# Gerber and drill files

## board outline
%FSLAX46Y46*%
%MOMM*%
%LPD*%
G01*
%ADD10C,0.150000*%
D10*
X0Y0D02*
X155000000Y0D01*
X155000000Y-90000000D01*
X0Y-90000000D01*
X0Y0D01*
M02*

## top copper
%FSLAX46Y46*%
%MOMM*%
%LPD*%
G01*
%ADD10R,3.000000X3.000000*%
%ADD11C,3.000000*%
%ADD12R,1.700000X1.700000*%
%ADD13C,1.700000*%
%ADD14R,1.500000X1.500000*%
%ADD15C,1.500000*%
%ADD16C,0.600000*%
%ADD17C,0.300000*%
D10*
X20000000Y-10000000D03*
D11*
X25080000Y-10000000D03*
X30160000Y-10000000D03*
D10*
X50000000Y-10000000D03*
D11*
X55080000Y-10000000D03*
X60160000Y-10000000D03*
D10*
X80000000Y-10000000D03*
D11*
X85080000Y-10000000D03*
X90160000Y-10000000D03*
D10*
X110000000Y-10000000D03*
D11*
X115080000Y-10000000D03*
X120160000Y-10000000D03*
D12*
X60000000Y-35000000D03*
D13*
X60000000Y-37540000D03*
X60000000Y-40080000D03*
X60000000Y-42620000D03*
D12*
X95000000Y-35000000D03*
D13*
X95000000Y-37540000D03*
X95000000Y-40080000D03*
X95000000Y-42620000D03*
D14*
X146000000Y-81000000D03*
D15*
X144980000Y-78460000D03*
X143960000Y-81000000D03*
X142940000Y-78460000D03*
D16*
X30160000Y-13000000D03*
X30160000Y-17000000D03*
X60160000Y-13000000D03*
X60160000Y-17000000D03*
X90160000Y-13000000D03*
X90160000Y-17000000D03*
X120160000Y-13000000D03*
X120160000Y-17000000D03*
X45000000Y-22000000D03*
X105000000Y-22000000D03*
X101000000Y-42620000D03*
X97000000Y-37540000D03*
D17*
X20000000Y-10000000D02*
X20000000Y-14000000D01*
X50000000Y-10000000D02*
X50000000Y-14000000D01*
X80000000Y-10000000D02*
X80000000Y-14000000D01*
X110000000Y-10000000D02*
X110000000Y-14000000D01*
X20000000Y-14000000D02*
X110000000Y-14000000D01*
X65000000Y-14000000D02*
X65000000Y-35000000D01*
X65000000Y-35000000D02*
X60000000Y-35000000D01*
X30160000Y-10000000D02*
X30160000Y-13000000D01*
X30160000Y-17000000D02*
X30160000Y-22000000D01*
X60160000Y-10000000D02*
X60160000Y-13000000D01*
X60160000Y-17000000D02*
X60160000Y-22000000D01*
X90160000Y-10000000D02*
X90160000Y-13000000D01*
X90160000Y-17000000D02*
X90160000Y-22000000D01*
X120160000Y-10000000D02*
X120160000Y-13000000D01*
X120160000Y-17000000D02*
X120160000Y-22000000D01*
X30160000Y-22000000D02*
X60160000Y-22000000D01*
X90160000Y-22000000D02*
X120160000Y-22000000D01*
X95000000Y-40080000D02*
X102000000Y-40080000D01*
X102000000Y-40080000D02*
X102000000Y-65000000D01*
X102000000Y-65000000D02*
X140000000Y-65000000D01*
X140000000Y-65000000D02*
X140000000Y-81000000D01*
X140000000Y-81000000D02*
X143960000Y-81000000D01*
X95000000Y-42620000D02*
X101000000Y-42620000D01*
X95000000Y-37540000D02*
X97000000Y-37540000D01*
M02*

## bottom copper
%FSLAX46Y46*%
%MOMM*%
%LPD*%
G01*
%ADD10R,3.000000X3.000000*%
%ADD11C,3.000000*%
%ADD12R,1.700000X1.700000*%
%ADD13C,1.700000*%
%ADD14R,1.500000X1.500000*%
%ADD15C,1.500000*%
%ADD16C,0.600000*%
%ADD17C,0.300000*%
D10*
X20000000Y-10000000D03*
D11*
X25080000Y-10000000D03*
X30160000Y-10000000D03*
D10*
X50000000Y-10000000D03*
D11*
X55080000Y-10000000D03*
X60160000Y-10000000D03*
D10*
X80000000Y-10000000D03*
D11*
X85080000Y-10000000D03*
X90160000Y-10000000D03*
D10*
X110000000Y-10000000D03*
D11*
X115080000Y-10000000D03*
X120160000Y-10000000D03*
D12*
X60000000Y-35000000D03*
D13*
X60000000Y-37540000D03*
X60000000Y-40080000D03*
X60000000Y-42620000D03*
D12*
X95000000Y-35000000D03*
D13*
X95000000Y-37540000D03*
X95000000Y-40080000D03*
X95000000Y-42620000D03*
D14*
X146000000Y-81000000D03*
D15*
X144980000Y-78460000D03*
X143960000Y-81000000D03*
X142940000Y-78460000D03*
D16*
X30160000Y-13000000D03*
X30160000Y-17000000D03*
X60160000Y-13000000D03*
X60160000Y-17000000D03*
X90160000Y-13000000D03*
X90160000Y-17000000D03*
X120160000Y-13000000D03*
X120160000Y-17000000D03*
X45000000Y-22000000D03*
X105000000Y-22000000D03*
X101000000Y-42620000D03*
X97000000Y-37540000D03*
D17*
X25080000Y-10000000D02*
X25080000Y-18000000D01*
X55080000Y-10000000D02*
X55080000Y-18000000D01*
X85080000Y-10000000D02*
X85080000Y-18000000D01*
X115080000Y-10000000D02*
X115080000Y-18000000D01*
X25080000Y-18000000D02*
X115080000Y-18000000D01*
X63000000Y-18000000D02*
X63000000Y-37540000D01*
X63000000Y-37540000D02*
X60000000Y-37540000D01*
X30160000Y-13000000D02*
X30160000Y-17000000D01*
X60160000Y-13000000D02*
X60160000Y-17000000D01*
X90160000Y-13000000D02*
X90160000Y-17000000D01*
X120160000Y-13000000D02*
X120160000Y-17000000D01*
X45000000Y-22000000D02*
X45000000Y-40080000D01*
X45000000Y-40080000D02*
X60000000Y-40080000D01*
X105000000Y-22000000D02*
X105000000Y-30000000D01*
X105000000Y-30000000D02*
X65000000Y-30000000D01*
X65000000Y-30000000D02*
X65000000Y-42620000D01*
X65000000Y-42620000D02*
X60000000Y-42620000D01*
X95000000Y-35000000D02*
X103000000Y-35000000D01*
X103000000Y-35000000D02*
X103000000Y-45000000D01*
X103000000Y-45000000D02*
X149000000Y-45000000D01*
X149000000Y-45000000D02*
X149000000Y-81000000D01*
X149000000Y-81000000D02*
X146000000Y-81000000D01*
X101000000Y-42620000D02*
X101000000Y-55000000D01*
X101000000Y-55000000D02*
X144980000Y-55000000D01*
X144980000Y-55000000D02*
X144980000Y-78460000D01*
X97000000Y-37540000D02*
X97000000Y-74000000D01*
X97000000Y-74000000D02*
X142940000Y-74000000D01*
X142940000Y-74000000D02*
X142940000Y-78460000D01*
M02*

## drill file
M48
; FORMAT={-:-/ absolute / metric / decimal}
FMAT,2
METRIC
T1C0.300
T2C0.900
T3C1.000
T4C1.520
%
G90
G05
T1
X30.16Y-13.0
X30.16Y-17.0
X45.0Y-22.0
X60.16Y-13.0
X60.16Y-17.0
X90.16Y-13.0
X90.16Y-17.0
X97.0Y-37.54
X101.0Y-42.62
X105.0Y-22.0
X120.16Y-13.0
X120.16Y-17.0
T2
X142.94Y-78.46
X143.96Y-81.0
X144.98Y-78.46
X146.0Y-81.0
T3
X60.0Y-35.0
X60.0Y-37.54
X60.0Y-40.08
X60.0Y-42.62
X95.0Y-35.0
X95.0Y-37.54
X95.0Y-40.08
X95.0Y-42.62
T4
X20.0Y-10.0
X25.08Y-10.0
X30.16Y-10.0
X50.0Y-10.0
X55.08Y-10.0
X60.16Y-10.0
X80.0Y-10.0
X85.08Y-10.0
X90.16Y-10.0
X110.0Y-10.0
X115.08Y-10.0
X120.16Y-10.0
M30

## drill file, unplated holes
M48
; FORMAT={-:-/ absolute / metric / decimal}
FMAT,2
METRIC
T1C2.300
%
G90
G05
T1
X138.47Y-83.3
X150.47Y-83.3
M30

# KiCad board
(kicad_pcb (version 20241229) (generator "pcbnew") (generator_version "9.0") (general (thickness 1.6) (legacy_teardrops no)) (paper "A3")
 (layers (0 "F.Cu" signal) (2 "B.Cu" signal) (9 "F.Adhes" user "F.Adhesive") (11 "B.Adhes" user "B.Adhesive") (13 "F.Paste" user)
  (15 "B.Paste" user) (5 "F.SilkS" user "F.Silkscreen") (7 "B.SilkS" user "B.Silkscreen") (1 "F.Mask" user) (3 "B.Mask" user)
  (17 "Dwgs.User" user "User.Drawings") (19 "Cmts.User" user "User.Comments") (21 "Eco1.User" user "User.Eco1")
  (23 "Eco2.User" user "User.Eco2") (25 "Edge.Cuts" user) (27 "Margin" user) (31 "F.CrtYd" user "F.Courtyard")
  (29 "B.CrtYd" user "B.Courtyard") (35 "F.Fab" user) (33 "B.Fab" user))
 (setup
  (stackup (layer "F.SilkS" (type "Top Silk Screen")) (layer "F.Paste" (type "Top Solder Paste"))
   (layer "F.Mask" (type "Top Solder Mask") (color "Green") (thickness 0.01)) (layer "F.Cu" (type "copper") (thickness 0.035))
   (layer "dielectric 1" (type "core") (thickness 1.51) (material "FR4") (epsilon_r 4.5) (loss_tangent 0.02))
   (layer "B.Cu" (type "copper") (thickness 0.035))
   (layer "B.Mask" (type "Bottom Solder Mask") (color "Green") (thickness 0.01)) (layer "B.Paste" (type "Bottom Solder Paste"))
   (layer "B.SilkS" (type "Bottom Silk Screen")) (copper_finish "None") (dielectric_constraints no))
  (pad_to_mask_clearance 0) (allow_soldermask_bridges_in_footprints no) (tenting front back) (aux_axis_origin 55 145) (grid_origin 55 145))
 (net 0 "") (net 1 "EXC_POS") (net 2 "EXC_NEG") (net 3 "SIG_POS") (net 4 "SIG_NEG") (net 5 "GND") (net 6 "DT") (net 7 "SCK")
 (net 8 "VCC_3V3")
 (gr_rect (start 0 0) (end 155 90) (stroke (width 0.15) (type solid)) (fill no) (layer "Edge.Cuts"))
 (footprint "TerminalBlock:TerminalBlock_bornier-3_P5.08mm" (layer "F.Cu") (at 20 10 0) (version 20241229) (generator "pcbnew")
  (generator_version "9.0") (layer "F.Cu")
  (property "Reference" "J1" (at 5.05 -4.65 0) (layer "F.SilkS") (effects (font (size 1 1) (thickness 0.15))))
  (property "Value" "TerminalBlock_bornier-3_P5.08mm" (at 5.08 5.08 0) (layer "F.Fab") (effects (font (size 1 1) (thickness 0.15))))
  (pad "1" thru_hole rect (at 0 0) (size 3 3) (drill 1.52) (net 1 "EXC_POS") (layers "*.Cu" "*.Mask") (remove_unused_layers no))
  (pad "2" thru_hole circle (at 5.08 0) (size 3 3) (drill 1.52) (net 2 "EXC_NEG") (layers "*.Cu" "*.Mask") (remove_unused_layers no))
  (pad "3" thru_hole circle (at 10.16 0) (size 3 3) (drill 1.52) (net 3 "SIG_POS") (layers "*.Cu" "*.Mask") (remove_unused_layers no)))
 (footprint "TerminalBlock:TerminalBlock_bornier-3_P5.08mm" (layer "F.Cu") (at 50 10 0) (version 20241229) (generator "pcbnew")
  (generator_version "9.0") (layer "F.Cu")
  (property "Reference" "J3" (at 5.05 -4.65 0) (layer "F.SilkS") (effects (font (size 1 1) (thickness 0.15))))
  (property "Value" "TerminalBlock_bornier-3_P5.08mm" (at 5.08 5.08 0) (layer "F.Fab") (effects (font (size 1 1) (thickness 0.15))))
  (pad "1" thru_hole rect (at 0 0) (size 3 3) (drill 1.52) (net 1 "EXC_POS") (layers "*.Cu" "*.Mask") (remove_unused_layers no))
  (pad "2" thru_hole circle (at 5.08 0) (size 3 3) (drill 1.52) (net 2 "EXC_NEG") (layers "*.Cu" "*.Mask") (remove_unused_layers no))
  (pad "3" thru_hole circle (at 10.16 0) (size 3 3) (drill 1.52) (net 3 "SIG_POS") (layers "*.Cu" "*.Mask") (remove_unused_layers no)))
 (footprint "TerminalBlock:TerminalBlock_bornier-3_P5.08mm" (layer "F.Cu") (at 80 10 0) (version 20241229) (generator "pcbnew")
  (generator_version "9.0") (layer "F.Cu")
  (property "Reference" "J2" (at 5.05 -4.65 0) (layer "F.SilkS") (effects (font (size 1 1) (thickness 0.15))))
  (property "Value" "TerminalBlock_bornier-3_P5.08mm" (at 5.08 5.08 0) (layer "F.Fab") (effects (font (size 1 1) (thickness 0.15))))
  (pad "1" thru_hole rect (at 0 0) (size 3 3) (drill 1.52) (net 1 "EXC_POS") (layers "*.Cu" "*.Mask") (remove_unused_layers no))
  (pad "2" thru_hole circle (at 5.08 0) (size 3 3) (drill 1.52) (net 2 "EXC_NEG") (layers "*.Cu" "*.Mask") (remove_unused_layers no))
  (pad "3" thru_hole circle (at 10.16 0) (size 3 3) (drill 1.52) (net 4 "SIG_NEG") (layers "*.Cu" "*.Mask") (remove_unused_layers no)))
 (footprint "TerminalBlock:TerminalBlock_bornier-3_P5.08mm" (layer "F.Cu") (at 110 10 0) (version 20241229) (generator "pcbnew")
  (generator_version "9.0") (layer "F.Cu")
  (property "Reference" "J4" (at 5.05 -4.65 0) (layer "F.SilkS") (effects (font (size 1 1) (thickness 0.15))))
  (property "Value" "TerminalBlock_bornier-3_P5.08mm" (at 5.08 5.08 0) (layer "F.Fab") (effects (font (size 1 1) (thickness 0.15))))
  (pad "1" thru_hole rect (at 0 0) (size 3 3) (drill 1.52) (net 1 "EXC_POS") (layers "*.Cu" "*.Mask") (remove_unused_layers no))
  (pad "2" thru_hole circle (at 5.08 0) (size 3 3) (drill 1.52) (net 2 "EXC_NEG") (layers "*.Cu" "*.Mask") (remove_unused_layers no))
  (pad "3" thru_hole circle (at 10.16 0) (size 3 3) (drill 1.52) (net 4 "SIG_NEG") (layers "*.Cu" "*.Mask") (remove_unused_layers no)))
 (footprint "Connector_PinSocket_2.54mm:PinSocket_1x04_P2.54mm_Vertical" (layer "F.Cu") (at 60 35 0) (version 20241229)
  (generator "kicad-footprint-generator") (layer "F.Cu")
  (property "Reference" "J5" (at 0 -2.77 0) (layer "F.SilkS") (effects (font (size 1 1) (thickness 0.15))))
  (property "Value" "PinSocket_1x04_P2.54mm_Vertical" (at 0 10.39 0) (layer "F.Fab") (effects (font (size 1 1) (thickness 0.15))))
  (pad "1" thru_hole rect (at 0 0) (size 1.7 1.7) (drill 1) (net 1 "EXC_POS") (layers "*.Cu" "*.Mask") (remove_unused_layers no))
  (pad "2" thru_hole circle (at 0 2.54) (size 1.7 1.7) (drill 1) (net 2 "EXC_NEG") (layers "*.Cu" "*.Mask") (remove_unused_layers no))
  (pad "3" thru_hole circle (at 0 5.08) (size 1.7 1.7) (drill 1) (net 3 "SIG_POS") (layers "*.Cu" "*.Mask") (remove_unused_layers no))
  (pad "4" thru_hole circle (at 0 7.62) (size 1.7 1.7) (drill 1) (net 4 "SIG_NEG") (layers "*.Cu" "*.Mask") (remove_unused_layers no)))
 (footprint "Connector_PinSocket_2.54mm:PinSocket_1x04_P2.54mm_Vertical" (layer "F.Cu") (at 95 35 0) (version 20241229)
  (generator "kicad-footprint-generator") (layer "F.Cu")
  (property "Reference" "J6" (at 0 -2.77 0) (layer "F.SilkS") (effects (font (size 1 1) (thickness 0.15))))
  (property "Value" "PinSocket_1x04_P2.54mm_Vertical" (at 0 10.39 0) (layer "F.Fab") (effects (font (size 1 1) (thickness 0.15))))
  (pad "1" thru_hole rect (at 0 0) (size 1.7 1.7) (drill 1) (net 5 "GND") (layers "*.Cu" "*.Mask") (remove_unused_layers no))
  (pad "2" thru_hole circle (at 0 2.54) (size 1.7 1.7) (drill 1) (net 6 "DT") (layers "*.Cu" "*.Mask") (remove_unused_layers no))
  (pad "3" thru_hole circle (at 0 5.08) (size 1.7 1.7) (drill 1) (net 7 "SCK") (layers "*.Cu" "*.Mask") (remove_unused_layers no))
  (pad "4" thru_hole circle (at 0 7.62) (size 1.7 1.7) (drill 1) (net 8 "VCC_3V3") (layers "*.Cu" "*.Mask") (remove_unused_layers no)))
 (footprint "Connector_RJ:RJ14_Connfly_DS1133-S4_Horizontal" (layer "F.Cu") (at 146 81 180) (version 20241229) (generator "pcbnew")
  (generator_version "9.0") (layer "F.Cu")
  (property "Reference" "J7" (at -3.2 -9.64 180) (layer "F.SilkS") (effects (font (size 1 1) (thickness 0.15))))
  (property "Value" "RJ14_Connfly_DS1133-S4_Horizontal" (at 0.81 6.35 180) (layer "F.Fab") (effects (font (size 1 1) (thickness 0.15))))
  (pad "" np_thru_hole circle (at -4.47 -2.3 180) (size 2.3 2.3) (drill 2.3) (layers "*.Cu" "*.Mask"))
  (pad "" np_thru_hole circle (at 7.53 -2.3 180) (size 2.3 2.3) (drill 2.3) (layers "*.Cu" "*.Mask"))
  (pad "1" thru_hole rect (at 0 0 180) (size 1.5 1.5) (drill 0.9) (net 5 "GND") (layers "*.Cu" "*.Mask") (remove_unused_layers no))
  (pad "2" thru_hole circle (at 1.02 2.54 180) (size 1.5 1.5) (drill 0.9) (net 8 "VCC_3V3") (layers "*.Cu" "*.Mask")
   (remove_unused_layers no))
  (pad "3" thru_hole circle (at 2.04 0 180) (size 1.5 1.5) (drill 0.9) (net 7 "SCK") (layers "*.Cu" "*.Mask") (remove_unused_layers no))
  (pad "4" thru_hole circle (at 3.06 2.54 180) (size 1.5 1.5) (drill 0.9) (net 6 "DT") (layers "*.Cu" "*.Mask") (remove_unused_layers no)))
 (segment (start 20 10) (end 20 14) (width 0.3) (layer "F.Cu") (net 1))
 (segment (start 50 10) (end 50 14) (width 0.3) (layer "F.Cu") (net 1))
 (segment (start 80 10) (end 80 14) (width 0.3) (layer "F.Cu") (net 1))
 (segment (start 110 10) (end 110 14) (width 0.3) (layer "F.Cu") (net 1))
 (segment (start 20 14) (end 110 14) (width 0.3) (layer "F.Cu") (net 1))
 (segment (start 65 14) (end 65 35) (width 0.3) (layer "F.Cu") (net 1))
 (segment (start 65 35) (end 60 35) (width 0.3) (layer "F.Cu") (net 1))
 (segment (start 25.08 10) (end 25.08 18) (width 0.3) (layer "B.Cu") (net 2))
 (segment (start 55.08 10) (end 55.08 18) (width 0.3) (layer "B.Cu") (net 2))
 (segment (start 85.08 10) (end 85.08 18) (width 0.3) (layer "B.Cu") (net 2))
 (segment (start 115.08 10) (end 115.08 18) (width 0.3) (layer "B.Cu") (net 2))
 (segment (start 25.08 18) (end 115.08 18) (width 0.3) (layer "B.Cu") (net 2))
 (segment (start 63 18) (end 63 37.54) (width 0.3) (layer "B.Cu") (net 2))
 (segment (start 63 37.54) (end 60 37.54) (width 0.3) (layer "B.Cu") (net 2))
 (segment (start 30.16 10) (end 30.16 13) (width 0.3) (layer "F.Cu") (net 3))
 (segment (start 30.16 13) (end 30.16 17) (width 0.3) (layer "B.Cu") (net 3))
 (segment (start 30.16 17) (end 30.16 22) (width 0.3) (layer "F.Cu") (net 3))
 (segment (start 60.16 10) (end 60.16 13) (width 0.3) (layer "F.Cu") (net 3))
 (segment (start 60.16 13) (end 60.16 17) (width 0.3) (layer "B.Cu") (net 3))
 (segment (start 60.16 17) (end 60.16 22) (width 0.3) (layer "F.Cu") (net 3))
 (segment (start 90.16 10) (end 90.16 13) (width 0.3) (layer "F.Cu") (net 4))
 (segment (start 90.16 13) (end 90.16 17) (width 0.3) (layer "B.Cu") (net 4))
 (segment (start 90.16 17) (end 90.16 22) (width 0.3) (layer "F.Cu") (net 4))
 (segment (start 120.16 10) (end 120.16 13) (width 0.3) (layer "F.Cu") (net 4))
 (segment (start 120.16 13) (end 120.16 17) (width 0.3) (layer "B.Cu") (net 4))
 (segment (start 120.16 17) (end 120.16 22) (width 0.3) (layer "F.Cu") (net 4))
 (segment (start 30.16 22) (end 60.16 22) (width 0.3) (layer "F.Cu") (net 3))
 (segment (start 90.16 22) (end 120.16 22) (width 0.3) (layer "F.Cu") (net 4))
 (segment (start 45 22) (end 45 40.08) (width 0.3) (layer "B.Cu") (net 3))
 (segment (start 45 40.08) (end 60 40.08) (width 0.3) (layer "B.Cu") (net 3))
 (segment (start 105 22) (end 105 30) (width 0.3) (layer "B.Cu") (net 4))
 (segment (start 105 30) (end 65 30) (width 0.3) (layer "B.Cu") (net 4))
 (segment (start 65 30) (end 65 42.62) (width 0.3) (layer "B.Cu") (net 4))
 (segment (start 65 42.62) (end 60 42.62) (width 0.3) (layer "B.Cu") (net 4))
 (segment (start 95 35) (end 103 35) (width 0.3) (layer "B.Cu") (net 5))
 (segment (start 103 35) (end 103 45) (width 0.3) (layer "B.Cu") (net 5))
 (segment (start 103 45) (end 149 45) (width 0.3) (layer "B.Cu") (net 5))
 (segment (start 149 45) (end 149 81) (width 0.3) (layer "B.Cu") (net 5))
 (segment (start 149 81) (end 146 81) (width 0.3) (layer "B.Cu") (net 5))
 (segment (start 95 40.08) (end 102 40.08) (width 0.3) (layer "F.Cu") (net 7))
 (segment (start 102 40.08) (end 102 65) (width 0.3) (layer "F.Cu") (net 7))
 (segment (start 102 65) (end 140 65) (width 0.3) (layer "F.Cu") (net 7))
 (segment (start 140 65) (end 140 81) (width 0.3) (layer "F.Cu") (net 7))
 (segment (start 140 81) (end 143.96 81) (width 0.3) (layer "F.Cu") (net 7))
 (segment (start 95 42.62) (end 101 42.62) (width 0.3) (layer "F.Cu") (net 8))
 (segment (start 101 42.62) (end 101 55) (width 0.3) (layer "B.Cu") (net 8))
 (segment (start 101 55) (end 144.98 55) (width 0.3) (layer "B.Cu") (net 8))
 (segment (start 144.98 55) (end 144.98 78.46) (width 0.3) (layer "B.Cu") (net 8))
 (segment (start 95 37.54) (end 97 37.54) (width 0.3) (layer "F.Cu") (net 6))
 (segment (start 97 37.54) (end 97 74) (width 0.3) (layer "B.Cu") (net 6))
 (segment (start 97 74) (end 142.94 74) (width 0.3) (layer "B.Cu") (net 6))
 (segment (start 142.94 74) (end 142.94 78.46) (width 0.3) (layer "B.Cu") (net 6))
 (via (at 30.16 13) (size 0.6) (drill 0.3) (layers "F.Cu" "B.Cu") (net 3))
 (via (at 30.16 17) (size 0.6) (drill 0.3) (layers "F.Cu" "B.Cu") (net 3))
 (via (at 60.16 13) (size 0.6) (drill 0.3) (layers "F.Cu" "B.Cu") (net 3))
 (via (at 60.16 17) (size 0.6) (drill 0.3) (layers "F.Cu" "B.Cu") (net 3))
 (via (at 90.16 13) (size 0.6) (drill 0.3) (layers "F.Cu" "B.Cu") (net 4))
 (via (at 90.16 17) (size 0.6) (drill 0.3) (layers "F.Cu" "B.Cu") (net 4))
 (via (at 120.16 13) (size 0.6) (drill 0.3) (layers "F.Cu" "B.Cu") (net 4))
 (via (at 120.16 17) (size 0.6) (drill 0.3) (layers "F.Cu" "B.Cu") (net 4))
 (via (at 45 22) (size 0.6) (drill 0.3) (layers "F.Cu" "B.Cu") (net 3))
 (via (at 105 22) (size 0.6) (drill 0.3) (layers "F.Cu" "B.Cu") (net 4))
 (via (at 101 42.62) (size 0.6) (drill 0.3) (layers "F.Cu" "B.Cu") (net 8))
 (via (at 97 37.54) (size 0.6) (drill 0.3) (layers "F.Cu" "B.Cu") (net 6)))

